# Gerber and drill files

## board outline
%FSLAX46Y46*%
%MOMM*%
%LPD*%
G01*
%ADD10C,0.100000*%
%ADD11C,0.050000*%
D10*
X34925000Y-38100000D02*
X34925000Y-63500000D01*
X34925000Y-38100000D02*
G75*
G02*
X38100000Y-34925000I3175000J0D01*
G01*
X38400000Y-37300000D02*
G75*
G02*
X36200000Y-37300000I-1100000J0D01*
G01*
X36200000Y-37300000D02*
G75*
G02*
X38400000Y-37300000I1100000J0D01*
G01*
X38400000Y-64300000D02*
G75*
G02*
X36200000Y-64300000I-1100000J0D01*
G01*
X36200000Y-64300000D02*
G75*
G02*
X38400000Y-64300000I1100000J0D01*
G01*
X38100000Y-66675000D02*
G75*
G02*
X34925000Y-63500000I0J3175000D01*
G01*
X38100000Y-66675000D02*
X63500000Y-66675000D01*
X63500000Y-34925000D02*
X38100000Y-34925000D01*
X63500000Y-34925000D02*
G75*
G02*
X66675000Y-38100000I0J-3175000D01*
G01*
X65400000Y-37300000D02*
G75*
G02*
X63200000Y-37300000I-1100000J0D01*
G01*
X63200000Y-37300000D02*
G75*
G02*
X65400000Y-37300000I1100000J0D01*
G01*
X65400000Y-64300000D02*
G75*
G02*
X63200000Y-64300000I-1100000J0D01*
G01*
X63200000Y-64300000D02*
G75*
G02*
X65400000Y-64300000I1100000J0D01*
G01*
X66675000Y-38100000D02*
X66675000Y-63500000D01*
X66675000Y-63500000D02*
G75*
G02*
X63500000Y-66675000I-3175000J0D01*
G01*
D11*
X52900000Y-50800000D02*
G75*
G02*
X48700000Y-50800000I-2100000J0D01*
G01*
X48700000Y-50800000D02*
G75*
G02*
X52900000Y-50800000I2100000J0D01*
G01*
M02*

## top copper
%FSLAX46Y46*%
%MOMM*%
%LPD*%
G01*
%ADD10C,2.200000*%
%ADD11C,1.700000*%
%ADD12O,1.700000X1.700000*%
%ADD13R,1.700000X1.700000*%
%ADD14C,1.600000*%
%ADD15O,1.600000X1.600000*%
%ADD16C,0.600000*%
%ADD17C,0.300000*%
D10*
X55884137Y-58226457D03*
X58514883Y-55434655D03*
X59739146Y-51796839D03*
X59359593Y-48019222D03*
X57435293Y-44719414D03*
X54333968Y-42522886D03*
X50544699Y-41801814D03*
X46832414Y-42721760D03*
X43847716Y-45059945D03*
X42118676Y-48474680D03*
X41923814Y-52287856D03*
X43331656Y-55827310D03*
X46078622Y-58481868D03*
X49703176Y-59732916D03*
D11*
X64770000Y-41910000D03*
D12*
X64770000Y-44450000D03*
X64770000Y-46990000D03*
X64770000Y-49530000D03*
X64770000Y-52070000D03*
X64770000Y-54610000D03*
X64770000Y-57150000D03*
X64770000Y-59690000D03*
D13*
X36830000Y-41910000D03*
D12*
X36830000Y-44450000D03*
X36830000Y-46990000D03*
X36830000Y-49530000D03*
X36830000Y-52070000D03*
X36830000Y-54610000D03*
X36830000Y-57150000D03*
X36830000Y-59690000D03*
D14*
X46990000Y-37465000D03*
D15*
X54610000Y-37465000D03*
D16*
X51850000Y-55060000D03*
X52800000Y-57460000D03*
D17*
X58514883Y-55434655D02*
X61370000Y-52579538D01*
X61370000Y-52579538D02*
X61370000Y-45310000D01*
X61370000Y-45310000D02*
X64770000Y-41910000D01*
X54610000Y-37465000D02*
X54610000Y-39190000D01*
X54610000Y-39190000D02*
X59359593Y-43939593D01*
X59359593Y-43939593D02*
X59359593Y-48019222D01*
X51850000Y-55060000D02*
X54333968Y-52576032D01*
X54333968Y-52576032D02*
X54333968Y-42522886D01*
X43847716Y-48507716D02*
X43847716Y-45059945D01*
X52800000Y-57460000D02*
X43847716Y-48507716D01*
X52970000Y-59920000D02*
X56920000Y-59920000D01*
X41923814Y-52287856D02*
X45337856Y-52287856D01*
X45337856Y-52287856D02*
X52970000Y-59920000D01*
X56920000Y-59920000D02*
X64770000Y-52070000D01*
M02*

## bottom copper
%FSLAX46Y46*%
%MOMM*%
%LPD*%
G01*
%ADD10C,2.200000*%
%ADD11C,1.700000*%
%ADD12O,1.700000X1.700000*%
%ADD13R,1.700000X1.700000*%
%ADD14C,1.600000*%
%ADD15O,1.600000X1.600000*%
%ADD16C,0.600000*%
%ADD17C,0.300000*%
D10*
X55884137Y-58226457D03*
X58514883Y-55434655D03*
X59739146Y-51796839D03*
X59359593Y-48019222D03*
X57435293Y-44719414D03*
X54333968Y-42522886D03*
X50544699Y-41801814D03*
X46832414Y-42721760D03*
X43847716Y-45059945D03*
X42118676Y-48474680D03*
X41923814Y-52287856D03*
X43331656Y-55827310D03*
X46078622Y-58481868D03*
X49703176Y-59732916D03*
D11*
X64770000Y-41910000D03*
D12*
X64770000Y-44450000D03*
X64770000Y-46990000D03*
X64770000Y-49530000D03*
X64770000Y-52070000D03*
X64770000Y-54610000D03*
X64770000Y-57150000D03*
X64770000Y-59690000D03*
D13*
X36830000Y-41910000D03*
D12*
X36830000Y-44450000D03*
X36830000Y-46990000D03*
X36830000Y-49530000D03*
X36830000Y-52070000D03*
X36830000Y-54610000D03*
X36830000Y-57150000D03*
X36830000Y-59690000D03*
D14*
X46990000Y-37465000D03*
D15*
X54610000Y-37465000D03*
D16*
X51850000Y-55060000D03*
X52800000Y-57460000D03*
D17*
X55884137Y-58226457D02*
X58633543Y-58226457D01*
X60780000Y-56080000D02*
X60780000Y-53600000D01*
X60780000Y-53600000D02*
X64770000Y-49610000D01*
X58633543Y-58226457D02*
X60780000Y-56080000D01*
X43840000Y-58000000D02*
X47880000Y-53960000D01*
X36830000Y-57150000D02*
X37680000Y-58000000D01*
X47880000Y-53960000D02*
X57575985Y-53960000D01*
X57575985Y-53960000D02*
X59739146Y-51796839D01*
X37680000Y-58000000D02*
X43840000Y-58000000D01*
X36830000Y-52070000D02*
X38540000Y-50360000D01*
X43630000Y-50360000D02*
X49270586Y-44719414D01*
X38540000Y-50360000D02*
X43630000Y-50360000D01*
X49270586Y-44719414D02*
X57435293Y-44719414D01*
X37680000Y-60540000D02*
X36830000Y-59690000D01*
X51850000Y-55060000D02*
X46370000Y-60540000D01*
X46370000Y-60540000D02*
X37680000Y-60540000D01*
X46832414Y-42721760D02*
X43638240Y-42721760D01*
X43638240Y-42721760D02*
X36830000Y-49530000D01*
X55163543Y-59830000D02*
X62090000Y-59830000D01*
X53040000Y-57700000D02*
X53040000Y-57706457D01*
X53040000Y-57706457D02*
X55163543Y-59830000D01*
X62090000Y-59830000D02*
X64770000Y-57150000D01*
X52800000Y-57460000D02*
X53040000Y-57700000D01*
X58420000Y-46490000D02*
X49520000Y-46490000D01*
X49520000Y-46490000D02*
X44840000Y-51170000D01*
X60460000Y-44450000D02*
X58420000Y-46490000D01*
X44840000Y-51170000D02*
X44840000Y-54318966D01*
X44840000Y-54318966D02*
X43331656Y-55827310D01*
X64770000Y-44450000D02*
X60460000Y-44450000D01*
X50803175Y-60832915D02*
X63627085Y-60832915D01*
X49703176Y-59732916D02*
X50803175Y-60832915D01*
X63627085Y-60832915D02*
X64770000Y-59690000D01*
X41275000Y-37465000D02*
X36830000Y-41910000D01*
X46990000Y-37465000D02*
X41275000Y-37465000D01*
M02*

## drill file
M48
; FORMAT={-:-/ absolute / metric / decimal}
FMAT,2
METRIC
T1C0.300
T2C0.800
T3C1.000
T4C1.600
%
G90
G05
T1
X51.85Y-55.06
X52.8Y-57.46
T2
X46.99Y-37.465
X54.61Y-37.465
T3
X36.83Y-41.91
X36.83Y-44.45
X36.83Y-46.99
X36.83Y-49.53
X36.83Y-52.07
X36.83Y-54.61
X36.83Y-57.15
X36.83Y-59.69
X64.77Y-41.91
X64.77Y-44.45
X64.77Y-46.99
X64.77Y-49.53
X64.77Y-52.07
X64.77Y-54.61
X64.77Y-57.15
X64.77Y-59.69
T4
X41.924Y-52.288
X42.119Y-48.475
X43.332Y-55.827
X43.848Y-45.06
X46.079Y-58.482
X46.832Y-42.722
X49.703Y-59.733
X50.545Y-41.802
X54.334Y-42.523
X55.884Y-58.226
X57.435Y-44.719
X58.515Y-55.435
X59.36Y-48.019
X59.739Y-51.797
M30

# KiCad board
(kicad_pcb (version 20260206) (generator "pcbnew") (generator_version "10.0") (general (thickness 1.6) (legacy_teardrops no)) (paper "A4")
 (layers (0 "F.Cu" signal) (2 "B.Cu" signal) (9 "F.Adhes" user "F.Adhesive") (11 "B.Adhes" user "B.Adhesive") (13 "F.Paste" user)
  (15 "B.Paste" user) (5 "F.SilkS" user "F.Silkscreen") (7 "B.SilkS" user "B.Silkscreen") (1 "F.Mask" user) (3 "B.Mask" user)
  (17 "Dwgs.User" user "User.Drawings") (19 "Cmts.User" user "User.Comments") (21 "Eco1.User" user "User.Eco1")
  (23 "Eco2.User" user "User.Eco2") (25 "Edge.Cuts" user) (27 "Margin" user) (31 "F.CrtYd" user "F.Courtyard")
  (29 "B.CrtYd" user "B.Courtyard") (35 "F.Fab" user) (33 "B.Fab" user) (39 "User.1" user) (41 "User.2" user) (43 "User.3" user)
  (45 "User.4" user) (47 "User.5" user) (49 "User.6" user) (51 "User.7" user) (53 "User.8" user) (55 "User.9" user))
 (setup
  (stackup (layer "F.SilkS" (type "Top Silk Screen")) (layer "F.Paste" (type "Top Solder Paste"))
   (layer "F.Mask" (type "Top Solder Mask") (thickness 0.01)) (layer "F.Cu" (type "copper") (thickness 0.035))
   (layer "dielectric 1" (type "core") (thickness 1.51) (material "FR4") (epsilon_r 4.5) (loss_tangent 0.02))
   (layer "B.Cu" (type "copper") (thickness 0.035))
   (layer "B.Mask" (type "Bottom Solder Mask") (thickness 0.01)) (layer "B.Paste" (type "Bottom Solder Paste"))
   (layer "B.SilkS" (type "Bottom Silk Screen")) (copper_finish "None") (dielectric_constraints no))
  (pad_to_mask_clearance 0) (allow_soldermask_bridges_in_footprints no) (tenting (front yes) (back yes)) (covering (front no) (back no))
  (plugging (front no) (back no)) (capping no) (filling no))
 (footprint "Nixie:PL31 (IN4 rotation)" (layer "F.Cu") (at 50.8 50.8)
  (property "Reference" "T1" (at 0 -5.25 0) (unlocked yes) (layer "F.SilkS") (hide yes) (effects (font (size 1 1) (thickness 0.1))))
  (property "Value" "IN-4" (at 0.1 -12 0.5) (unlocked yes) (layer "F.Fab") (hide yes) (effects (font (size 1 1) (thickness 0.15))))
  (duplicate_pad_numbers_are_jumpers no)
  (fp_circle (center 0 0) (end 2.09928 -0.054972) (stroke (width 0.05) (type default)) (fill no) (layer "Edge.Cuts"))
  (pad "1" thru_hole circle (at 5.084137 7.426457 173) (size 2.2 2.2) (drill 1.6) (layers "*.Cu" "*.Mask") (remove_unused_layers no)
   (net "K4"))
  (pad "2" thru_hole circle (at 7.714883 4.634655 173) (size 2.2 2.2) (drill 1.6) (layers "*.Cu" "*.Mask") (remove_unused_layers no)
   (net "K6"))
  (pad "3" thru_hole circle (at 8.939146 0.996839 173) (size 2.2 2.2) (drill 1.6) (layers "*.Cu" "*.Mask") (remove_unused_layers no)
   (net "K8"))
  (pad "4" thru_hole circle (at 8.559593 -2.780778 173) (size 2.2 2.2) (drill 1.6) (layers "*.Cu" "*.Mask") (remove_unused_layers no)
   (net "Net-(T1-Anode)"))
  (pad "5" thru_hole circle (at 6.635293 -6.080586 173) (size 2.2 2.2) (drill 1.6) (layers "*.Cu" "*.Mask") (remove_unused_layers no)
   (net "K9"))
  (pad "6" thru_hole circle (at 3.533968 -8.277114 173) (size 2.2 2.2) (drill 1.6) (layers "*.Cu" "*.Mask") (remove_unused_layers no)
   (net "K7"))
  (pad "7" thru_hole circle (at -0.255301 -8.998186 173) (size 2.2 2.2) (drill 1.6) (layers "*.Cu" "*.Mask") (remove_unused_layers no)
   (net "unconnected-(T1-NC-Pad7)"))
  (pad "8" thru_hole circle (at -3.967586 -8.07824 173) (size 2.2 2.2) (drill 1.6) (layers "*.Cu" "*.Mask") (remove_unused_layers no)
   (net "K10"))
  (pad "9" thru_hole circle (at -6.952284 -5.740055 173) (size 2.2 2.2) (drill 1.6) (layers "*.Cu" "*.Mask") (remove_unused_layers no)
   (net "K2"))
  (pad "10" thru_hole circle (at -8.681324 -2.32532 173) (size 2.2 2.2) (drill 1.6) (layers "*.Cu" "*.Mask") (remove_unused_layers no)
   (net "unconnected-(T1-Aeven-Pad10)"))
  (pad "11" thru_hole circle (at -8.876186 1.487856 173) (size 2.2 2.2) (drill 1.6) (layers "*.Cu" "*.Mask") (remove_unused_layers no)
   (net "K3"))
  (pad "12" thru_hole circle (at -7.468344 5.02731 173) (size 2.2 2.2) (drill 1.6) (layers "*.Cu" "*.Mask") (remove_unused_layers no)
   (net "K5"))
  (pad "13" thru_hole circle (at -4.721378 7.681868 173) (size 2.2 2.2) (drill 1.6) (layers "*.Cu" "*.Mask") (remove_unused_layers no)
   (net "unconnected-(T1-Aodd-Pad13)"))
  (pad "14" thru_hole circle (at -1.096824 8.932916 173) (size 2.2 2.2) (drill 1.6) (layers "*.Cu" "*.Mask") (remove_unused_layers no)
   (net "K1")))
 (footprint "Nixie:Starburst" (layer "F.Cu") (at 43 63.25)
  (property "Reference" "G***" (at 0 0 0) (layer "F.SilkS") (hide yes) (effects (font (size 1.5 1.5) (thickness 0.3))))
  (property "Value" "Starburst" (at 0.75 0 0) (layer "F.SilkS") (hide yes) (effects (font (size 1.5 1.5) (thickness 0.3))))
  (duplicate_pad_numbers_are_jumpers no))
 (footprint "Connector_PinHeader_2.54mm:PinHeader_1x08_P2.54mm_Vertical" (layer "B.Cu") (at 64.77 41.91 180)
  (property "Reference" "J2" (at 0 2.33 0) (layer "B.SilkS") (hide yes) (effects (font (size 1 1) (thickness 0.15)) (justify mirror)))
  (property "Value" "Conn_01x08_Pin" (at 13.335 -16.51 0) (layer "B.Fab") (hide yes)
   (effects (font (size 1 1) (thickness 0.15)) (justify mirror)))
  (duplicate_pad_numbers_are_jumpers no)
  (pad "1" thru_hole circle (at 0 0 180) (size 1.7 1.7) (drill 1) (layers "*.Cu" "*.Mask") (remove_unused_layers no) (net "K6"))
  (pad "2" thru_hole oval (at 0 -2.54 180) (size 1.7 1.7) (drill 1) (layers "*.Cu" "*.Mask") (remove_unused_layers no) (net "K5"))
  (pad "3" thru_hole oval (at 0 -5.08 180) (size 1.7 1.7) (drill 1) (layers "*.Cu" "*.Mask") (remove_unused_layers no)
   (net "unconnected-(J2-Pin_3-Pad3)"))
  (pad "4" thru_hole oval (at 0 -7.62 180) (size 1.7 1.7) (drill 1) (layers "*.Cu" "*.Mask") (remove_unused_layers no) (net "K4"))
  (pad "5" thru_hole oval (at 0 -10.16 180) (size 1.7 1.7) (drill 1) (layers "*.Cu" "*.Mask") (remove_unused_layers no) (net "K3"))
  (pad "6" thru_hole oval (at 0 -12.7 180) (size 1.7 1.7) (drill 1) (layers "*.Cu" "*.Mask") (remove_unused_layers no)
   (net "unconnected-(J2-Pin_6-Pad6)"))
  (pad "7" thru_hole oval (at 0 -15.24 180) (size 1.7 1.7) (drill 1) (layers "*.Cu" "*.Mask") (remove_unused_layers no) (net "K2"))
  (pad "8" thru_hole oval (at 0 -17.78 180) (size 1.7 1.7) (drill 1) (layers "*.Cu" "*.Mask") (remove_unused_layers no) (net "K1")))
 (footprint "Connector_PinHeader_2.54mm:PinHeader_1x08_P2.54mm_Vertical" (layer "B.Cu") (at 36.83 41.91 180)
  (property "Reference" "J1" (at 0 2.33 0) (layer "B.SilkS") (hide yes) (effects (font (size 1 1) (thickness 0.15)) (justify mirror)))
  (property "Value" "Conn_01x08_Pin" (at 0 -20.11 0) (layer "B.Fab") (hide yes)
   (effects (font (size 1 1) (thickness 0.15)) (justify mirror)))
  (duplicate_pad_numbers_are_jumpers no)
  (pad "1" thru_hole rect (at 0 0 180) (size 1.7 1.7) (drill 1) (layers "*.Cu" "*.Mask") (remove_unused_layers no) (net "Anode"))
  (pad "2" thru_hole oval (at 0 -2.54 180) (size 1.7 1.7) (drill 1) (layers "*.Cu" "*.Mask") (remove_unused_layers no)
   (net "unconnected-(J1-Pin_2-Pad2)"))
  (pad "3" thru_hole oval (at 0 -5.08 180) (size 1.7 1.7) (drill 1) (layers "*.Cu" "*.Mask") (remove_unused_layers no)
   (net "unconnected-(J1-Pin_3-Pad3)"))
  (pad "4" thru_hole oval (at 0 -7.62 180) (size 1.7 1.7) (drill 1) (layers "*.Cu" "*.Mask") (remove_unused_layers no) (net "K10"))
  (pad "5" thru_hole oval (at 0 -10.16 180) (size 1.7 1.7) (drill 1) (layers "*.Cu" "*.Mask") (remove_unused_layers no) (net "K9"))
  (pad "6" thru_hole oval (at 0 -12.7 180) (size 1.7 1.7) (drill 1) (layers "*.Cu" "*.Mask") (remove_unused_layers no)
   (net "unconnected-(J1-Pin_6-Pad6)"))
  (pad "7" thru_hole oval (at 0 -15.24 180) (size 1.7 1.7) (drill 1) (layers "*.Cu" "*.Mask") (remove_unused_layers no) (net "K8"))
  (pad "8" thru_hole oval (at 0 -17.78 180) (size 1.7 1.7) (drill 1) (layers "*.Cu" "*.Mask") (remove_unused_layers no) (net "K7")))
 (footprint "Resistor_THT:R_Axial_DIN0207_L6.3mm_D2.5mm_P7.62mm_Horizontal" (layer "B.Cu") (at 46.99 37.465)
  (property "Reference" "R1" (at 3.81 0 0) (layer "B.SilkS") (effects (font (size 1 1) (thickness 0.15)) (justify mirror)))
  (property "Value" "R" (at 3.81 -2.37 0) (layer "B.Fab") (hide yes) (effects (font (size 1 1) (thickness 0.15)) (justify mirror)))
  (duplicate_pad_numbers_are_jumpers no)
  (pad "1" thru_hole circle (at 0 0) (size 1.6 1.6) (drill 0.8) (layers "*.Cu" "*.Mask") (remove_unused_layers no) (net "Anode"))
  (pad "2" thru_hole oval (at 7.62 0) (size 1.6 1.6) (drill 0.8) (layers "*.Cu" "*.Mask") (remove_unused_layers no) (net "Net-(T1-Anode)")))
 (gr_line (start 34.925 38.1) (end 34.925 63.5) (stroke (width 0.1) (type default)) (layer "Edge.Cuts"))
 (gr_arc (start 34.925 38.1) (mid 35.854936 35.854936) (end 38.1 34.925) (stroke (width 0.1) (type default)) (layer "Edge.Cuts"))
 (gr_circle (center 37.3 37.3) (end 38.4 37.3) (stroke (width 0.1) (type default)) (fill no) (layer "Edge.Cuts"))
 (gr_circle (center 37.3 64.3) (end 38.4 64.3) (stroke (width 0.1) (type default)) (fill no) (layer "Edge.Cuts"))
 (gr_arc (start 38.1 66.675) (mid 35.854936 65.745064) (end 34.925 63.5) (stroke (width 0.1) (type default)) (layer "Edge.Cuts"))
 (gr_line (start 38.1 66.675) (end 63.5 66.675) (stroke (width 0.1) (type default)) (layer "Edge.Cuts"))
 (gr_line (start 63.5 34.925) (end 38.1 34.925) (stroke (width 0.1) (type default)) (layer "Edge.Cuts"))
 (gr_arc (start 63.5 34.925) (mid 65.745064 35.854936) (end 66.675 38.1) (stroke (width 0.1) (type default)) (layer "Edge.Cuts"))
 (gr_circle (center 64.3 37.3) (end 65.4 37.3) (stroke (width 0.1) (type default)) (fill no) (layer "Edge.Cuts"))
 (gr_circle (center 64.3 64.3) (end 65.4 64.3) (stroke (width 0.1) (type default)) (fill no) (layer "Edge.Cuts"))
 (gr_line (start 66.675 38.1) (end 66.675 63.5) (stroke (width 0.1) (type default)) (layer "Edge.Cuts"))
 (gr_arc (start 66.675 63.5) (mid 65.745064 65.745064) (end 63.5 66.675) (stroke (width 0.1) (type default)) (layer "Edge.Cuts"))
 (segment (start 55.884137 58.226457) (end 58.633543 58.226457) (width 0.3) (layer "B.Cu") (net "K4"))
 (segment (start 60.78 56.08) (end 60.78 53.6) (width 0.3) (layer "B.Cu") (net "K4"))
 (segment (start 60.78 53.6) (end 64.77 49.61) (width 0.3) (layer "B.Cu") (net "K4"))
 (segment (start 58.633543 58.226457) (end 60.78 56.08) (width 0.3) (layer "B.Cu") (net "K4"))
 (segment (start 58.514883 55.434655) (end 61.37 52.579538) (width 0.3) (layer "F.Cu") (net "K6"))
 (segment (start 61.37 52.579538) (end 61.37 45.31) (width 0.3) (layer "F.Cu") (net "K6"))
 (segment (start 61.37 45.31) (end 64.77 41.91) (width 0.3) (layer "F.Cu") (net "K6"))
 (segment (start 43.84 58) (end 47.88 53.96) (width 0.3) (layer "B.Cu") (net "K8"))
 (segment (start 36.83 57.15) (end 37.68 58) (width 0.3) (layer "B.Cu") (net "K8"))
 (segment (start 47.88 53.96) (end 57.575985 53.96) (width 0.3) (layer "B.Cu") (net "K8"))
 (segment (start 57.575985 53.96) (end 59.739146 51.796839) (width 0.3) (layer "B.Cu") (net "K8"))
 (segment (start 37.68 58) (end 43.84 58) (width 0.3) (layer "B.Cu") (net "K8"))
 (segment (start 54.61 37.465) (end 54.61 39.19) (width 0.3) (layer "F.Cu") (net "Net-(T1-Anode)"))
 (segment (start 54.61 39.19) (end 59.359593 43.939593) (width 0.3) (layer "F.Cu") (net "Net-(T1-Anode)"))
 (segment (start 59.359593 43.939593) (end 59.359593 48.019222) (width 0.3) (layer "F.Cu") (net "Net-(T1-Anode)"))
 (segment (start 36.83 52.07) (end 38.54 50.36) (width 0.3) (layer "B.Cu") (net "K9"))
 (segment (start 43.63 50.36) (end 49.270586 44.719414) (width 0.3) (layer "B.Cu") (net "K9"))
 (segment (start 38.54 50.36) (end 43.63 50.36) (width 0.3) (layer "B.Cu") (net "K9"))
 (segment (start 49.270586 44.719414) (end 57.435293 44.719414) (width 0.3) (layer "B.Cu") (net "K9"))
 (segment (start 51.85 55.06) (end 54.333968 52.576032) (width 0.3) (layer "F.Cu") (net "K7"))
 (segment (start 54.333968 52.576032) (end 54.333968 42.522886) (width 0.3) (layer "F.Cu") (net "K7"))
 (via (at 51.85 55.06) (size 0.6) (drill 0.3) (layers "F.Cu" "B.Cu") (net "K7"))
 (segment (start 37.68 60.54) (end 36.83 59.69) (width 0.3) (layer "B.Cu") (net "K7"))
 (segment (start 51.85 55.06) (end 46.37 60.54) (width 0.3) (layer "B.Cu") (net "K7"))
 (segment (start 46.37 60.54) (end 37.68 60.54) (width 0.3) (layer "B.Cu") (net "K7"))
 (segment (start 46.832414 42.72176) (end 43.63824 42.72176) (width 0.3) (layer "B.Cu") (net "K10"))
 (segment (start 43.63824 42.72176) (end 36.83 49.53) (width 0.3) (layer "B.Cu") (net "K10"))
 (segment (start 43.847716 48.507716) (end 43.847716 45.059945) (width 0.3) (layer "F.Cu") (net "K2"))
 (segment (start 52.8 57.46) (end 43.847716 48.507716) (width 0.3) (layer "F.Cu") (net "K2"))
 (via (at 52.8 57.46) (size 0.6) (drill 0.3) (layers "F.Cu" "B.Cu") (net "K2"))
 (segment (start 55.163543 59.83) (end 62.09 59.83) (width 0.3) (layer "B.Cu") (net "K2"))
 (segment (start 53.04 57.7) (end 53.04 57.706457) (width 0.3) (layer "B.Cu") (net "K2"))
 (segment (start 53.04 57.706457) (end 55.163543 59.83) (width 0.3) (layer "B.Cu") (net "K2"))
 (segment (start 62.09 59.83) (end 64.77 57.15) (width 0.3) (layer "B.Cu") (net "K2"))
 (segment (start 52.8 57.46) (end 53.04 57.7) (width 0.3) (layer "B.Cu") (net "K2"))
 (segment (start 52.97 59.92) (end 56.92 59.92) (width 0.3) (layer "F.Cu") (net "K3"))
 (segment (start 41.923814 52.287856) (end 45.337856 52.287856) (width 0.3) (layer "F.Cu") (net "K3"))
 (segment (start 45.337856 52.287856) (end 52.97 59.92) (width 0.3) (layer "F.Cu") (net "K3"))
 (segment (start 56.92 59.92) (end 64.77 52.07) (width 0.3) (layer "F.Cu") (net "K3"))
 (segment (start 58.42 46.49) (end 49.52 46.49) (width 0.3) (layer "B.Cu") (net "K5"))
 (segment (start 49.52 46.49) (end 44.84 51.17) (width 0.3) (layer "B.Cu") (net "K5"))
 (segment (start 60.46 44.45) (end 58.42 46.49) (width 0.3) (layer "B.Cu") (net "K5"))
 (segment (start 44.84 51.17) (end 44.84 54.318966) (width 0.3) (layer "B.Cu") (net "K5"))
 (segment (start 44.84 54.318966) (end 43.331656 55.82731) (width 0.3) (layer "B.Cu") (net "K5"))
 (segment (start 64.77 44.45) (end 60.46 44.45) (width 0.3) (layer "B.Cu") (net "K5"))
 (segment (start 50.803175 60.832915) (end 63.627085 60.832915) (width 0.3) (layer "B.Cu") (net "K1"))
 (segment (start 49.703176 59.732916) (end 50.803175 60.832915) (width 0.3) (layer "B.Cu") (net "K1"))
 (segment (start 63.627085 60.832915) (end 64.77 59.69) (width 0.3) (layer "B.Cu") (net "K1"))
 (segment (start 41.275 37.465) (end 36.83 41.91) (width 0.3) (layer "B.Cu") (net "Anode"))
 (segment (start 46.99 37.465) (end 41.275 37.465) (width 0.3) (layer "B.Cu") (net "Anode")))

